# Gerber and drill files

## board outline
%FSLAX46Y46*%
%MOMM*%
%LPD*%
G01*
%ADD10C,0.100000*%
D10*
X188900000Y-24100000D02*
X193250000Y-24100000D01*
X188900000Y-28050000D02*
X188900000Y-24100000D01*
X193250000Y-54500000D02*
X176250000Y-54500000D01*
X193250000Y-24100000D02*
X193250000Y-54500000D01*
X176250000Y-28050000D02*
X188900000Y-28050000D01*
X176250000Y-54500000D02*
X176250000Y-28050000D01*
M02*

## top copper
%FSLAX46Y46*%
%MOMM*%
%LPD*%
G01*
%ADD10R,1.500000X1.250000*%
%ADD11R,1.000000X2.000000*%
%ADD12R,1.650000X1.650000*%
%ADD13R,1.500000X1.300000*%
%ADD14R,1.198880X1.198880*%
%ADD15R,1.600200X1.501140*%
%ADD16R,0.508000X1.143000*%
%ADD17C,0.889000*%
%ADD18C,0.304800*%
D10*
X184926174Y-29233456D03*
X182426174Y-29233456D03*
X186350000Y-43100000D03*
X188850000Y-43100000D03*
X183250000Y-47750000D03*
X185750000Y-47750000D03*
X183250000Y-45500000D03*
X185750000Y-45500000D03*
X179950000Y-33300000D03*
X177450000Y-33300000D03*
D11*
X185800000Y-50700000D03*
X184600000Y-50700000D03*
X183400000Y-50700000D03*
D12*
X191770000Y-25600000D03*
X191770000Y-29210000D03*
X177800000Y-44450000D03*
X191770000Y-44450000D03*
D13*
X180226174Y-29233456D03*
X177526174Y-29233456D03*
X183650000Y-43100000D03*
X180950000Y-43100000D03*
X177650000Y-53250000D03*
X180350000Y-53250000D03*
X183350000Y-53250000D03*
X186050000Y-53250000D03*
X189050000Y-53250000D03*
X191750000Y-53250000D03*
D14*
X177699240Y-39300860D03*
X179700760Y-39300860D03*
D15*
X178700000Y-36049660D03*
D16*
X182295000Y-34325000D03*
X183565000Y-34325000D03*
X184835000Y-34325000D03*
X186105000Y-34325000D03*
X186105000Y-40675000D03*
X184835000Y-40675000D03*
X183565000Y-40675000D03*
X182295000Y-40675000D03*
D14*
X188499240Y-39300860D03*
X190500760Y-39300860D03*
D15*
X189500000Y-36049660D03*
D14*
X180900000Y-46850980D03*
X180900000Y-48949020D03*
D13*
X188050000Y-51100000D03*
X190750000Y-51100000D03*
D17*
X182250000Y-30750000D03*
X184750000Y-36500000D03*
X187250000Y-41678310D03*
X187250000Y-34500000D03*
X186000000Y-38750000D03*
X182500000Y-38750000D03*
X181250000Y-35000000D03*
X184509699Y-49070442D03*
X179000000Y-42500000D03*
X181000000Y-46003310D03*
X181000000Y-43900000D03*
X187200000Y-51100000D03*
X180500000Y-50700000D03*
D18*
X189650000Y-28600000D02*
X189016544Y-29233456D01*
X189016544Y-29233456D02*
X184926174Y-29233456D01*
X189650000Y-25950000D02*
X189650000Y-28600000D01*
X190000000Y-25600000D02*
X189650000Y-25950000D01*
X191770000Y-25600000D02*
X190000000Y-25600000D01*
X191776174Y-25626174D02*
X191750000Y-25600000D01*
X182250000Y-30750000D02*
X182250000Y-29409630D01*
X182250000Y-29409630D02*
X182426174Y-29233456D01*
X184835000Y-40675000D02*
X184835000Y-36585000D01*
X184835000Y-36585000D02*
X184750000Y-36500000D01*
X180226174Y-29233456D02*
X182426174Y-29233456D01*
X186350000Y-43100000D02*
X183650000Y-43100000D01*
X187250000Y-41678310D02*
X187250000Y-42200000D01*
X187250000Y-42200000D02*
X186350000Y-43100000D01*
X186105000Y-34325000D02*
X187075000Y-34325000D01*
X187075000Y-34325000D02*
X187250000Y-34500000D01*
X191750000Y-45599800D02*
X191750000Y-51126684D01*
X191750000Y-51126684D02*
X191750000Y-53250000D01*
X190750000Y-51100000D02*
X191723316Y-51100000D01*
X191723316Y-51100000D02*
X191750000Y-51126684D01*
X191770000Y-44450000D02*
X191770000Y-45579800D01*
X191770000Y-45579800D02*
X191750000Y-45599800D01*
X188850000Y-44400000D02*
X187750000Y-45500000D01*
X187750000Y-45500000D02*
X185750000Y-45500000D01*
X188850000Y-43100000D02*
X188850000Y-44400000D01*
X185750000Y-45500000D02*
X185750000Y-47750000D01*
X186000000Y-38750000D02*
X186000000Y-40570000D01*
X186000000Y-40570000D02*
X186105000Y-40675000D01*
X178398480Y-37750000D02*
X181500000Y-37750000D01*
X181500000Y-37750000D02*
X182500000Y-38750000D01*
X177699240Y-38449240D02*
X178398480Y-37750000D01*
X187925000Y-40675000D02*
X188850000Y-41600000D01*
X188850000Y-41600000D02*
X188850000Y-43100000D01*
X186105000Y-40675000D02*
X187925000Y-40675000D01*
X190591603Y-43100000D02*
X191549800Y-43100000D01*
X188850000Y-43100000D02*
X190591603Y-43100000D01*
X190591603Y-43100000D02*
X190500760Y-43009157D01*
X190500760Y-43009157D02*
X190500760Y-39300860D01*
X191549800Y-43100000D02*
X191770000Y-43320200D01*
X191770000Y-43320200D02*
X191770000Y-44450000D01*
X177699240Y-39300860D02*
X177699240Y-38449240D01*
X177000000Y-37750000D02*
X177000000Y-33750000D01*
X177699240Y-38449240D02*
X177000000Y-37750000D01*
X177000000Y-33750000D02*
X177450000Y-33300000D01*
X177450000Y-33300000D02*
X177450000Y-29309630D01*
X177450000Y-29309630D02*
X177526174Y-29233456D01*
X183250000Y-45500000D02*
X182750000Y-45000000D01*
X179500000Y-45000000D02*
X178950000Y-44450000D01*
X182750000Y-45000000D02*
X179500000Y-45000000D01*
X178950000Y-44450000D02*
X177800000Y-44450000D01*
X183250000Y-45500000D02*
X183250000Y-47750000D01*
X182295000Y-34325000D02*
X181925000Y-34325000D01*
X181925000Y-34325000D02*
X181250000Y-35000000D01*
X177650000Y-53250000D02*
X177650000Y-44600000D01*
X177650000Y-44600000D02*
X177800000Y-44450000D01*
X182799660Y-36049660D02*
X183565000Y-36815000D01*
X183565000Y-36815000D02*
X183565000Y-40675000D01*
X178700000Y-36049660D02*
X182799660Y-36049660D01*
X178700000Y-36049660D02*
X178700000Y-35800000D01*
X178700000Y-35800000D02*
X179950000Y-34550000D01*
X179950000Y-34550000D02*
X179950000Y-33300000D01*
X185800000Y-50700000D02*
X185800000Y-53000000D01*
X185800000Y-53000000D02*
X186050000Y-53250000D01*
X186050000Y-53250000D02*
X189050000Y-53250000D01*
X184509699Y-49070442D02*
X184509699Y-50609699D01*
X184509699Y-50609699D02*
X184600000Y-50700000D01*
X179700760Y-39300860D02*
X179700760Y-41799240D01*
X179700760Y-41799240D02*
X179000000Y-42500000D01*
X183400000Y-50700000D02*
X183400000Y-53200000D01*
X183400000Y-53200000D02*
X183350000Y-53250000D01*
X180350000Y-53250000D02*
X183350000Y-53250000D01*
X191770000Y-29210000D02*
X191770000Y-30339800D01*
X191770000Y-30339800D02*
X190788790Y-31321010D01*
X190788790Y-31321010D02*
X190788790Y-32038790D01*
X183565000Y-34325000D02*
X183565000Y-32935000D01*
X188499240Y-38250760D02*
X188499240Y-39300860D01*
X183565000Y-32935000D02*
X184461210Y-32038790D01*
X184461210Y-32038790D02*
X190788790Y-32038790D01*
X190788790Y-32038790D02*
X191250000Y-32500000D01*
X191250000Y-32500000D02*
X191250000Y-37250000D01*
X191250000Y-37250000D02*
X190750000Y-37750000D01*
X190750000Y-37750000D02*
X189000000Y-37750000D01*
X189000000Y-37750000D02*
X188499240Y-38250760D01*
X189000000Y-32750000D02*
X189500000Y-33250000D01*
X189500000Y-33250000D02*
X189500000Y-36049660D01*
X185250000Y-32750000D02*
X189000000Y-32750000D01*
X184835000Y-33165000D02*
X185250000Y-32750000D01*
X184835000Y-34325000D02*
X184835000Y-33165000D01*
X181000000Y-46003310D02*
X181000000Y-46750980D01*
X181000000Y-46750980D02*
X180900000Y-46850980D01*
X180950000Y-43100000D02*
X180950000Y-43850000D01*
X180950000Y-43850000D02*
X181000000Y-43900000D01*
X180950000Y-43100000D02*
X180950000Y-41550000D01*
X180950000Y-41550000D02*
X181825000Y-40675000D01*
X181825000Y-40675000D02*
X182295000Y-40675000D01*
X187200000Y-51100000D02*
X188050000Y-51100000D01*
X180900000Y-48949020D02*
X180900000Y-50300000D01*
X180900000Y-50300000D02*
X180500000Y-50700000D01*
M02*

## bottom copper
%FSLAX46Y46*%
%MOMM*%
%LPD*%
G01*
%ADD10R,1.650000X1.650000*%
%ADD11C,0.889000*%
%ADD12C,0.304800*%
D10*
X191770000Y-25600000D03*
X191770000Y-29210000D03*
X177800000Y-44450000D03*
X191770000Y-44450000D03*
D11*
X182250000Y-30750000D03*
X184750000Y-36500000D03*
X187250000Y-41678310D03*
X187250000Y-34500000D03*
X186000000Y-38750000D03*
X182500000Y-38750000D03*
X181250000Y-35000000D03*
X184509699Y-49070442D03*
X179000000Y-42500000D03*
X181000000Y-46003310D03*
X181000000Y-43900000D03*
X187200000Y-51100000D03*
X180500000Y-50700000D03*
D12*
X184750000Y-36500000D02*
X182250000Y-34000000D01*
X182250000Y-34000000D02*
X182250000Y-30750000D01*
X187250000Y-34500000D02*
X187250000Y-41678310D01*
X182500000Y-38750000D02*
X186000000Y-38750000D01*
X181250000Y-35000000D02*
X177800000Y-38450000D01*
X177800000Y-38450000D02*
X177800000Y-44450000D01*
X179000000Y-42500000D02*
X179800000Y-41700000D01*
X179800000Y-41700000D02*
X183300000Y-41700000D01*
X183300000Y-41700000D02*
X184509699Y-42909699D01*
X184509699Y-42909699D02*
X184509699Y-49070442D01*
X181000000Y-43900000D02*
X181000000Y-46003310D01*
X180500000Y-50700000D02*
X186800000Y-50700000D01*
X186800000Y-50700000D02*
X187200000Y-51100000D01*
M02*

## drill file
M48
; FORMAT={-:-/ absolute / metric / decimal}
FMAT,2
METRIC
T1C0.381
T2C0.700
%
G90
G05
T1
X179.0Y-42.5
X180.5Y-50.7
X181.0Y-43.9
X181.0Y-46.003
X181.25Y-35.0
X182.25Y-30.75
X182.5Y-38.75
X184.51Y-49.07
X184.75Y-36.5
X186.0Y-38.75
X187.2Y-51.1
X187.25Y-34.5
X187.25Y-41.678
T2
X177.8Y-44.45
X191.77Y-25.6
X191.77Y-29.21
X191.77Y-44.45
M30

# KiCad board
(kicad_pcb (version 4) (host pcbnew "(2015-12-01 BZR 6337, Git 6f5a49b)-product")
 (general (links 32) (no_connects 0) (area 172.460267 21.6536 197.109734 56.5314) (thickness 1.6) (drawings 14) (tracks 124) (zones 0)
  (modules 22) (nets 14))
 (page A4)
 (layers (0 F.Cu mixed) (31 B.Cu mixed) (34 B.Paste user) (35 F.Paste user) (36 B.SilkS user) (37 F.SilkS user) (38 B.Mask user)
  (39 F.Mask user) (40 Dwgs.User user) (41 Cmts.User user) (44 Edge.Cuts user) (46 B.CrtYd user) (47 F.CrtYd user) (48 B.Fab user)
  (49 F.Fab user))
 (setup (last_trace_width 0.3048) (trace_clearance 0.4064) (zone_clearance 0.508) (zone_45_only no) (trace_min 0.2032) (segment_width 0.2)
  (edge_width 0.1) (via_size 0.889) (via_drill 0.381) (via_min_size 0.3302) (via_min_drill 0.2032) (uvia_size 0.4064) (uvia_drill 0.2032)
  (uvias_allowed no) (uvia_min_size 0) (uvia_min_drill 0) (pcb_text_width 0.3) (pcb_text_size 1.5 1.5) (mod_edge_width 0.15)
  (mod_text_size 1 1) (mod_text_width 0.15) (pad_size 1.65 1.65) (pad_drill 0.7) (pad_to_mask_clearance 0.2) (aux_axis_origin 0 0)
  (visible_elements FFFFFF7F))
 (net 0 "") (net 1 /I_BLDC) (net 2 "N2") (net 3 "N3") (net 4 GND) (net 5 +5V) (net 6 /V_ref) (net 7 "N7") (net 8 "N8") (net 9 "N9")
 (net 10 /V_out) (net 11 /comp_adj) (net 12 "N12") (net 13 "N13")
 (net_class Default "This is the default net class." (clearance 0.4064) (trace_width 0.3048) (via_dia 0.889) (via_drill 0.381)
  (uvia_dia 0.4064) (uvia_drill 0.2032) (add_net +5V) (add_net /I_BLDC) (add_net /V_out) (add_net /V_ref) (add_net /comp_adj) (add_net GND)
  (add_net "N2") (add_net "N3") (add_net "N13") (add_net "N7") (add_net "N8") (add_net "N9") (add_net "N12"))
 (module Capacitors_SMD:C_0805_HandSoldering (layer F.Cu) (at 183.676174 29.233456 180)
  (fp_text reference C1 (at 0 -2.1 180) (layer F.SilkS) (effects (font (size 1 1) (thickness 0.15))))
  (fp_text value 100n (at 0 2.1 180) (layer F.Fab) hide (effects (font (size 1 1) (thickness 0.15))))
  (pad 1 smd rect (at -1.25 0 180) (size 1.5 1.25) (layers F.Cu F.Paste F.Mask) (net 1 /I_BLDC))
  (pad 2 smd rect (at 1.25 0 180) (size 1.5 1.25) (layers F.Cu F.Paste F.Mask) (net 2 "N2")))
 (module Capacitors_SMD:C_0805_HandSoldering (layer F.Cu) (at 187.6 43.1)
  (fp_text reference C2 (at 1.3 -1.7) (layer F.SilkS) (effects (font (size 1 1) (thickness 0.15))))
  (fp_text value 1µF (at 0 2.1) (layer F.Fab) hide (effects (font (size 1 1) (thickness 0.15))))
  (pad 1 smd rect (at -1.25 0) (size 1.5 1.25) (layers F.Cu F.Paste F.Mask) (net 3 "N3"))
  (pad 2 smd rect (at 1.25 0) (size 1.5 1.25) (layers F.Cu F.Paste F.Mask) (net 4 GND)))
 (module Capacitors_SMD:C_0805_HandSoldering (layer F.Cu) (at 184.5 47.75)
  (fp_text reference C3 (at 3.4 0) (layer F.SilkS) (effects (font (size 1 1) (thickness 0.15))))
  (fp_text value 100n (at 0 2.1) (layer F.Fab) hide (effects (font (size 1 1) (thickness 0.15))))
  (pad 1 smd rect (at -1.25 0) (size 1.5 1.25) (layers F.Cu F.Paste F.Mask) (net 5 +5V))
  (pad 2 smd rect (at 1.25 0) (size 1.5 1.25) (layers F.Cu F.Paste F.Mask) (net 4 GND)))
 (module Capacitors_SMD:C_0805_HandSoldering (layer F.Cu) (at 184.5 45.5)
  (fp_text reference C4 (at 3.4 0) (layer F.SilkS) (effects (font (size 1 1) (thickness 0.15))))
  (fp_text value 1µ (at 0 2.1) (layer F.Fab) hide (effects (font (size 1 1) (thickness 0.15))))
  (pad 1 smd rect (at -1.25 0) (size 1.5 1.25) (layers F.Cu F.Paste F.Mask) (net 5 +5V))
  (pad 2 smd rect (at 1.25 0) (size 1.5 1.25) (layers F.Cu F.Paste F.Mask) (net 4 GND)))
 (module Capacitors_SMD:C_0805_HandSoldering (layer F.Cu) (at 178.7 33.3 180)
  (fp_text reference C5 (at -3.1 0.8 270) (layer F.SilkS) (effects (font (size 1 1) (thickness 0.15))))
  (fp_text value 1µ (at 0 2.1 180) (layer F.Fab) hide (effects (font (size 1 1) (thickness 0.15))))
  (pad 1 smd rect (at -1.25 0 180) (size 1.5 1.25) (layers F.Cu F.Paste F.Mask) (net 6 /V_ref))
  (pad 2 smd rect (at 1.25 0 180) (size 1.5 1.25) (layers F.Cu F.Paste F.Mask) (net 4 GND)))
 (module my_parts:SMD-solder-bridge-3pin (layer F.Cu) (at 184.6 50.7 180) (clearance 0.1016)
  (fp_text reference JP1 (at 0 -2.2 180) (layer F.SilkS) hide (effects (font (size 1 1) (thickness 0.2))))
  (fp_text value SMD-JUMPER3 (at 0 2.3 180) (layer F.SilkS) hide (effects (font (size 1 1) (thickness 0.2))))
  (pad 1 smd rect (at -1.2 0 180) (size 1 2) (layers F.Cu F.Mask) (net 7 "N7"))
  (pad 2 smd rect (at 0 0 180) (size 1 2) (layers F.Cu F.Mask) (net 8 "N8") (solder_mask_margin 0.3))
  (pad 3 smd rect (at 1.2 0 180) (size 1 2) (layers F.Cu F.Mask) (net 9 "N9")))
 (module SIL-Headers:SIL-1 (layer F.Cu) (at 191.77 25.6)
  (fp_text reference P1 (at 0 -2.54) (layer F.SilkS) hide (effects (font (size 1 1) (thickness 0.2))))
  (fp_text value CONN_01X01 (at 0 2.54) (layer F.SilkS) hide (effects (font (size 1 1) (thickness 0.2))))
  (pad 1 thru_hole rect (at 0 0) (size 1.65 1.65) (drill 0.7) (layers *.Cu *.Mask) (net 1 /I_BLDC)))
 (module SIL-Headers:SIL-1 (layer F.Cu) (at 191.77 29.21)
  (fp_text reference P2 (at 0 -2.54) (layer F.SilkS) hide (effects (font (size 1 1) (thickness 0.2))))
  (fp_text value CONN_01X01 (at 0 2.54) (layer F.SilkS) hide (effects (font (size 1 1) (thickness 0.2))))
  (pad 1 thru_hole rect (at 0 0) (size 1.65 1.65) (drill 0.7) (layers *.Cu *.Mask) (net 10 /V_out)))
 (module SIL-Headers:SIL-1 (layer F.Cu) (at 177.8 44.45)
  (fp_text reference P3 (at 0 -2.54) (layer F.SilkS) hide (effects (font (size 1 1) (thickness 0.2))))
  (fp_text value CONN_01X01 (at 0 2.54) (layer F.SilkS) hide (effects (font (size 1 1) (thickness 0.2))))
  (pad 1 thru_hole rect (at 0 0) (size 1.65 1.65) (drill 0.7) (layers *.Cu *.Mask) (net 5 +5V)))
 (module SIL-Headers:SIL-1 (layer F.Cu) (at 191.77 44.45)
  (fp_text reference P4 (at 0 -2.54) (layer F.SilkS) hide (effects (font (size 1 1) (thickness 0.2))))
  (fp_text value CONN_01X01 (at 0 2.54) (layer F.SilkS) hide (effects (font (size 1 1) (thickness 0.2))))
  (pad 1 thru_hole rect (at 0 0) (size 1.65 1.65) (drill 0.7) (layers *.Cu *.Mask) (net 4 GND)))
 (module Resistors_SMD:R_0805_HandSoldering (layer F.Cu) (at 178.876174 29.233456 180)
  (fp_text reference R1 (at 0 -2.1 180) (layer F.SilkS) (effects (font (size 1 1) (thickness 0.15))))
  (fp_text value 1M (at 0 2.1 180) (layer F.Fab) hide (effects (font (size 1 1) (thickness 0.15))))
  (pad 1 smd rect (at -1.35 0 180) (size 1.5 1.3) (layers F.Cu F.Paste F.Mask) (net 2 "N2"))
  (pad 2 smd rect (at 1.35 0 180) (size 1.5 1.3) (layers F.Cu F.Paste F.Mask) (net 4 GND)))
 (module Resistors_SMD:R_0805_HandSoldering (layer F.Cu) (at 182.3 43.1 180)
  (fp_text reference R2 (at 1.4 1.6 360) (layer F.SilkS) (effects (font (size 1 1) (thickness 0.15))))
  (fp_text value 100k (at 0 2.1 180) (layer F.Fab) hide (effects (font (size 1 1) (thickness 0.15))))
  (pad 1 smd rect (at -1.35 0 180) (size 1.5 1.3) (layers F.Cu F.Paste F.Mask) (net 3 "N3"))
  (pad 2 smd rect (at 1.35 0 180) (size 1.5 1.3) (layers F.Cu F.Paste F.Mask) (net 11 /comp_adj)))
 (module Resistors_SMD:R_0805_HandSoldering (layer F.Cu) (at 179 53.25)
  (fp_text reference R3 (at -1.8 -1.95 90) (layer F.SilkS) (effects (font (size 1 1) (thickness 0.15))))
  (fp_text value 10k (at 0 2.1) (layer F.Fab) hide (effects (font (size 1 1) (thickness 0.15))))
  (pad 1 smd rect (at -1.35 0) (size 1.5 1.3) (layers F.Cu F.Paste F.Mask) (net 5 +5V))
  (pad 2 smd rect (at 1.35 0) (size 1.5 1.3) (layers F.Cu F.Paste F.Mask) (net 9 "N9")))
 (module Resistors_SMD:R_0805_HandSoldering (layer F.Cu) (at 184.7 53.25)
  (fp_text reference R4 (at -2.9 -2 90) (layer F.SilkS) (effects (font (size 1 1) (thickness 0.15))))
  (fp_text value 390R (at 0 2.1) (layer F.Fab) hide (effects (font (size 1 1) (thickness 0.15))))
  (pad 1 smd rect (at -1.35 0) (size 1.5 1.3) (layers F.Cu F.Paste F.Mask) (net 9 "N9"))
  (pad 2 smd rect (at 1.35 0) (size 1.5 1.3) (layers F.Cu F.Paste F.Mask) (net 7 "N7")))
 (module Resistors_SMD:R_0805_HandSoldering (layer F.Cu) (at 190.4 53.25)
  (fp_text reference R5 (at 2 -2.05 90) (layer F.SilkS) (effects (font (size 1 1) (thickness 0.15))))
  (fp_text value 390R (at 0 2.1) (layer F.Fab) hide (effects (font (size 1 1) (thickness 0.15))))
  (pad 1 smd rect (at -1.35 0) (size 1.5 1.3) (layers F.Cu F.Paste F.Mask) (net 7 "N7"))
  (pad 2 smd rect (at 1.35 0) (size 1.5 1.3) (layers F.Cu F.Paste F.Mask) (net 4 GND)))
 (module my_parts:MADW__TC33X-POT (layer F.Cu) (at 178.7 37.5)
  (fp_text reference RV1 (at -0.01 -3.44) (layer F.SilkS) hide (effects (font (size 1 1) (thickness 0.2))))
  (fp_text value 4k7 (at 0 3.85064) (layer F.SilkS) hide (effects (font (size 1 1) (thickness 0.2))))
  (pad 1 smd rect (at -1.00076 1.80086) (size 1.19888 1.19888) (layers F.Cu F.Paste F.Mask) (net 4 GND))
  (pad 3 smd rect (at 1.00076 1.80086) (size 1.19888 1.19888) (layers F.Cu F.Paste F.Mask) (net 8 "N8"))
  (pad 2 smd rect (at 0 -1.45034) (size 1.6002 1.50114) (layers F.Cu F.Paste F.Mask) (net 6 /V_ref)))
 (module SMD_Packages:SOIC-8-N (layer F.Cu) (at 184.2 37.5)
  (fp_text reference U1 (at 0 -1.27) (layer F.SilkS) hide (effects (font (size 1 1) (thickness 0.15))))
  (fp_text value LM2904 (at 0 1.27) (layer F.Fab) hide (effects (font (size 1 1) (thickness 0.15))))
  (pad 8 smd rect (at -1.905 -3.175) (size 0.508 1.143) (layers F.Cu F.Paste F.Mask) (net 5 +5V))
  (pad 7 smd rect (at -0.635 -3.175) (size 0.508 1.143) (layers F.Cu F.Paste F.Mask) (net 10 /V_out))
  (pad 6 smd rect (at 0.635 -3.175) (size 0.508 1.143) (layers F.Cu F.Paste F.Mask) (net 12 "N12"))
  (pad 5 smd rect (at 1.905 -3.175) (size 0.508 1.143) (layers F.Cu F.Paste F.Mask) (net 3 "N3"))
  (pad 4 smd rect (at 1.905 3.175) (size 0.508 1.143) (layers F.Cu F.Paste F.Mask) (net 4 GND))
  (pad 3 smd rect (at 0.635 3.175) (size 0.508 1.143) (layers F.Cu F.Paste F.Mask) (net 2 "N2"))
  (pad 2 smd rect (at -0.635 3.175) (size 0.508 1.143) (layers F.Cu F.Paste F.Mask) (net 6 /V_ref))
  (pad 1 smd rect (at -1.905 3.175) (size 0.508 1.143) (layers F.Cu F.Paste F.Mask) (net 11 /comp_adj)))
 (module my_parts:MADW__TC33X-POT (layer F.Cu) (at 189.5 37.5)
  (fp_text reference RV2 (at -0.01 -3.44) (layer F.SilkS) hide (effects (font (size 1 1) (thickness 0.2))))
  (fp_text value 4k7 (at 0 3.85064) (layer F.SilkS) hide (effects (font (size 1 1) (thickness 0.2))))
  (pad 1 smd rect (at -1.00076 1.80086) (size 1.19888 1.19888) (layers F.Cu F.Paste F.Mask) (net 10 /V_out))
  (pad 3 smd rect (at 1.00076 1.80086) (size 1.19888 1.19888) (layers F.Cu F.Paste F.Mask) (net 4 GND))
  (pad 2 smd rect (at 0 -1.45034) (size 1.6002 1.50114) (layers F.Cu F.Paste F.Mask) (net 12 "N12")))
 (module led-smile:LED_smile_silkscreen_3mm (layer F.Cu) (at 186.85 31.85)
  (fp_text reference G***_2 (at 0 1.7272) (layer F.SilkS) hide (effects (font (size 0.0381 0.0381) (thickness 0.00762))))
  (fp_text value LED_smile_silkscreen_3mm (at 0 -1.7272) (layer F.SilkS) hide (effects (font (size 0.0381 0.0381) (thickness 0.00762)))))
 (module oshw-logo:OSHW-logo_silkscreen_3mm (layer F.Cu) (at 191.7 41.45)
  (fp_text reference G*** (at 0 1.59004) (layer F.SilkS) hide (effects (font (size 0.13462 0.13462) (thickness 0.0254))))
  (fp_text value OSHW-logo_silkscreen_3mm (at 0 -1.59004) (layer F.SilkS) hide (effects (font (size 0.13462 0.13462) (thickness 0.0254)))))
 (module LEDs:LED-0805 (layer F.Cu) (at 180.9 47.9 90)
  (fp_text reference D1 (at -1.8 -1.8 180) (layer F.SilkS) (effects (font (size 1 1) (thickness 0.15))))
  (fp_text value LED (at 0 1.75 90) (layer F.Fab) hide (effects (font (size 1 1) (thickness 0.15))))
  (pad 2 smd rect (at 1.04902 0 270) (size 1.19888 1.19888) (layers F.Cu F.Paste F.Mask) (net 11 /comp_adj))
  (pad 1 smd rect (at -1.04902 0 270) (size 1.19888 1.19888) (layers F.Cu F.Paste F.Mask) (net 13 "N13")))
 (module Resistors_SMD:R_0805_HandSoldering (layer F.Cu) (at 189.4 51.1)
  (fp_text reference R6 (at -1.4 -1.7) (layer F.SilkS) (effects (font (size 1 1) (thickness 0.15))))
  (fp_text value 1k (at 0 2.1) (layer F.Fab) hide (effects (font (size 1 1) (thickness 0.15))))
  (pad 1 smd rect (at -1.35 0) (size 1.5 1.3) (layers F.Cu F.Paste F.Mask) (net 13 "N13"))
  (pad 2 smd rect (at 1.35 0) (size 1.5 1.3) (layers F.Cu F.Paste F.Mask) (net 4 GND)))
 (gr_line (start 188.9 24.1) (end 193.25 24.1) (layer Edge.Cuts) (width 0.1))
 (gr_line (start 188.9 28.05) (end 188.9 24.1) (layer Edge.Cuts) (width 0.1))
 (gr_line (start 193.25 54.5) (end 176.25 54.5) (layer Edge.Cuts) (width 0.1))
 (gr_line (start 193.25 24.1) (end 193.25 54.5) (layer Edge.Cuts) (width 0.1))
 (gr_line (start 176.25 28.05) (end 188.9 28.05) (layer Edge.Cuts) (width 0.1))
 (gr_line (start 176.25 54.5) (end 176.25 28.05) (layer Edge.Cuts) (width 0.1))
 (segment (start 189.65 28.6) (end 189.016544 29.233456) (width 0.3048) (layer F.Cu) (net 1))
 (segment (start 189.016544 29.233456) (end 184.926174 29.233456) (width 0.3048) (layer F.Cu) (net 1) (status 20))
 (segment (start 189.65 25.95) (end 189.65 28.6) (width 0.3048) (layer F.Cu) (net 1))
 (segment (start 190 25.6) (end 189.65 25.95) (width 0.3048) (layer F.Cu) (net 1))
 (segment (start 191.77 25.6) (end 190 25.6) (width 0.3048) (layer F.Cu) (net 1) (status 10))
 (segment (start 191.776174 25.626174) (end 191.75 25.6) (width 0.3048) (layer F.Cu) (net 1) (status 30))
 (segment (start 182.25 30.75) (end 182.25 29.40963) (width 0.3048) (layer F.Cu) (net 2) (status 20))
 (segment (start 182.25 29.40963) (end 182.426174 29.233456) (width 0.3048) (layer F.Cu) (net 2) (status 30))
 (segment (start 184.75 36.5) (end 182.25 34) (width 0.3048) (layer B.Cu) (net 2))
 (segment (start 182.25 34) (end 182.25 30.75) (width 0.3048) (layer B.Cu) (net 2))
 (segment (start 184.835 40.675) (end 184.835 36.585) (width 0.3048) (layer F.Cu) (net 2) (status 10))
 (segment (start 184.835 36.585) (end 184.75 36.5) (width 0.3048) (layer F.Cu) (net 2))
 (segment (start 180.226174 29.233456) (end 182.426174 29.233456) (width 0.3048) (layer F.Cu) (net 2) (status 30))
 (segment (start 186.35 43.1) (end 183.65 43.1) (width 0.3048) (layer F.Cu) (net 3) (status 30))
 (segment (start 187.25 41.67831) (end 187.25 42.2) (width 0.3048) (layer F.Cu) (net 3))
 (segment (start 187.25 42.2) (end 186.35 43.1) (width 0.3048) (layer F.Cu) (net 3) (status 20))
 (segment (start 187.25 34.5) (end 187.25 41.67831) (width 0.3048) (layer B.Cu) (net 3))
 (segment (start 186.105 34.325) (end 187.075 34.325) (width 0.3048) (layer F.Cu) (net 3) (status 10))
 (segment (start 187.075 34.325) (end 187.25 34.5) (width 0.3048) (layer F.Cu) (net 3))
 (segment (start 191.75 45.5998) (end 191.75 51.126684) (width 0.3048) (layer F.Cu) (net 4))
 (segment (start 191.75 51.126684) (end 191.75 53.25) (width 0.3048) (layer F.Cu) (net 4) (status 20))
 (segment (start 190.75 51.1) (end 191.723316 51.1) (width 0.3048) (layer F.Cu) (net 4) (status 10))
 (segment (start 191.723316 51.1) (end 191.75 51.126684) (width 0.3048) (layer F.Cu) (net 4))
 (segment (start 191.77 44.45) (end 191.77 45.5798) (width 0.3048) (layer F.Cu) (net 4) (status 10))
 (segment (start 191.77 45.5798) (end 191.75 45.5998) (width 0.3048) (layer F.Cu) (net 4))
 (segment (start 188.85 44.4) (end 187.75 45.5) (width 0.3048) (layer F.Cu) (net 4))
 (segment (start 187.75 45.5) (end 185.75 45.5) (width 0.3048) (layer F.Cu) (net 4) (status 20))
 (segment (start 188.85 43.1) (end 188.85 44.4) (width 0.3048) (layer F.Cu) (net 4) (status 10))
 (segment (start 185.75 45.5) (end 185.75 47.75) (width 0.3048) (layer F.Cu) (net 4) (status 30))
 (segment (start 186 38.75) (end 186 40.57) (width 0.3048) (layer F.Cu) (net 4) (status 20))
 (segment (start 186 40.57) (end 186.105 40.675) (width 0.3048) (layer F.Cu) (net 4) (status 30))
 (segment (start 182.5 38.75) (end 186 38.75) (width 0.3048) (layer B.Cu) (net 4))
 (segment (start 178.39848 37.75) (end 181.5 37.75) (width 0.3048) (layer F.Cu) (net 4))
 (segment (start 181.5 37.75) (end 182.5 38.75) (width 0.3048) (layer F.Cu) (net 4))
 (segment (start 177.69924 38.44924) (end 178.39848 37.75) (width 0.3048) (layer F.Cu) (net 4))
 (segment (start 187.925 40.675) (end 188.85 41.6) (width 0.3048) (layer F.Cu) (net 4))
 (segment (start 188.85 41.6) (end 188.85 43.1) (width 0.3048) (layer F.Cu) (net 4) (status 20))
 (segment (start 186.105 40.675) (end 187.925 40.675) (width 0.3048) (layer F.Cu) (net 4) (status 10))
 (segment (start 190.591603 43.1) (end 191.5498 43.1) (width 0.3048) (layer F.Cu) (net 4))
 (segment (start 188.85 43.1) (end 190.591603 43.1) (width 0.3048) (layer F.Cu) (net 4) (status 10))
 (segment (start 190.591603 43.1) (end 190.50076 43.009157) (width 0.3048) (layer F.Cu) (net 4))
 (segment (start 190.50076 43.009157) (end 190.50076 39.30086) (width 0.3048) (layer F.Cu) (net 4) (status 20))
 (segment (start 191.5498 43.1) (end 191.77 43.3202) (width 0.3048) (layer F.Cu) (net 4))
 (segment (start 191.77 43.3202) (end 191.77 44.45) (width 0.3048) (layer F.Cu) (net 4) (status 20))
 (segment (start 177.69924 39.30086) (end 177.69924 38.44924) (width 0.3048) (layer F.Cu) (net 4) (status 10))
 (segment (start 177 37.75) (end 177 33.75) (width 0.3048) (layer F.Cu) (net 4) (status 20))
 (segment (start 177.69924 38.44924) (end 177 37.75) (width 0.3048) (layer F.Cu) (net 4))
 (segment (start 177 33.75) (end 177.45 33.3) (width 0.3048) (layer F.Cu) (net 4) (status 30))
 (segment (start 177.45 33.3) (end 177.45 29.30963) (width 0.3048) (layer F.Cu) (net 4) (status 30))
 (segment (start 177.45 29.30963) (end 177.526174 29.233456) (width 0.3048) (layer F.Cu) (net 4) (status 30))
 (segment (start 183.25 45.5) (end 182.75 45) (width 0.3048) (layer F.Cu) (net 5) (status 30))
 (segment (start 179.5 45) (end 178.95 44.45) (width 0.3048) (layer F.Cu) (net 5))
 (segment (start 182.75 45) (end 179.5 45) (width 0.3048) (layer F.Cu) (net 5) (status 10))
 (segment (start 178.95 44.45) (end 177.8 44.45) (width 0.3048) (layer F.Cu) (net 5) (status 20))
 (segment (start 183.25 45.5) (end 183.25 47.75) (width 0.3048) (layer F.Cu) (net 5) (status 30))
 (segment (start 181.25 35) (end 177.8 38.45) (width 0.3048) (layer B.Cu) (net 5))
 (segment (start 177.8 38.45) (end 177.8 44.45) (width 0.3048) (layer B.Cu) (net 5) (status 20))
 (segment (start 182.295 34.325) (end 181.925 34.325) (width 0.3048) (layer F.Cu) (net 5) (status 10))
 (segment (start 181.925 34.325) (end 181.25 35) (width 0.3048) (layer F.Cu) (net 5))
 (segment (start 177.65 53.25) (end 177.65 44.6) (width 0.3048) (layer F.Cu) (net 5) (status 30))
 (segment (start 177.65 44.6) (end 177.8 44.45) (width 0.3048) (layer F.Cu) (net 5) (status 30))
 (segment (start 182.79966 36.04966) (end 183.565 36.815) (width 0.3048) (layer F.Cu) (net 6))
 (segment (start 183.565 36.815) (end 183.565 40.675) (width 0.3048) (layer F.Cu) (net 6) (status 20))
 (segment (start 178.7 36.04966) (end 182.79966 36.04966) (width 0.3048) (layer F.Cu) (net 6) (status 10))
 (segment (start 178.7 36.04966) (end 178.7 35.8) (width 0.3048) (layer F.Cu) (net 6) (status 30))
 (segment (start 178.7 35.8) (end 179.95 34.55) (width 0.3048) (layer F.Cu) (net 6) (status 10))
 (segment (start 179.95 34.55) (end 179.95 33.3) (width 0.3048) (layer F.Cu) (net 6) (status 20))
 (segment (start 185.8 50.7) (end 185.8 53) (width 0.3048) (layer F.Cu) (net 7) (status 30))
 (segment (start 185.8 53) (end 186.05 53.25) (width 0.3048) (layer F.Cu) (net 7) (status 30))
 (segment (start 186.05 53.25) (end 189.05 53.25) (width 0.3048) (layer F.Cu) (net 7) (status 30))
 (segment (start 179 42.5) (end 179.8 41.7) (width 0.3048) (layer B.Cu) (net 8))
 (segment (start 179.8 41.7) (end 183.3 41.7) (width 0.3048) (layer B.Cu) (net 8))
 (segment (start 183.3 41.7) (end 184.509699 42.909699) (width 0.3048) (layer B.Cu) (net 8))
 (segment (start 184.509699 42.909699) (end 184.509699 49.070442) (width 0.3048) (layer B.Cu) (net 8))
 (segment (start 184.509699 49.070442) (end 184.509699 50.609699) (width 0.3048) (layer F.Cu) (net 8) (status 20))
 (segment (start 184.509699 50.609699) (end 184.6 50.7) (width 0.3048) (layer F.Cu) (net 8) (status 30))
 (segment (start 179.70076 39.30086) (end 179.70076 41.79924) (width 0.3048) (layer F.Cu) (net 8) (status 10))
 (segment (start 179.70076 41.79924) (end 179 42.5) (width 0.3048) (layer F.Cu) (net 8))
 (segment (start 183.4 50.7) (end 183.4 53.2) (width 0.3048) (layer F.Cu) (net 9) (status 30))
 (segment (start 183.4 53.2) (end 183.35 53.25) (width 0.3048) (layer F.Cu) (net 9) (status 30))
 (segment (start 180.35 53.25) (end 183.35 53.25) (width 0.3048) (layer F.Cu) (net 9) (status 30))
 (segment (start 191.77 29.21) (end 191.77 30.3398) (width 0.3048) (layer F.Cu) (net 10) (status 10))
 (segment (start 191.77 30.3398) (end 190.78879 31.32101) (width 0.3048) (layer F.Cu) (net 10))
 (segment (start 190.78879 31.32101) (end 190.78879 32.03879) (width 0.3048) (layer F.Cu) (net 10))
 (segment (start 183.565 34.325) (end 183.565 32.935) (width 0.3048) (layer F.Cu) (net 10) (status 10))
 (segment (start 188.49924 38.25076) (end 188.49924 39.30086) (width 0.3048) (layer F.Cu) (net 10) (status 20))
 (segment (start 183.565 32.935) (end 184.46121 32.03879) (width 0.3048) (layer F.Cu) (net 10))
 (segment (start 184.46121 32.03879) (end 190.78879 32.03879) (width 0.3048) (layer F.Cu) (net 10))
 (segment (start 190.78879 32.03879) (end 191.25 32.5) (width 0.3048) (layer F.Cu) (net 10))
 (segment (start 191.25 32.5) (end 191.25 37.25) (width 0.3048) (layer F.Cu) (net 10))
 (segment (start 191.25 37.25) (end 190.75 37.75) (width 0.3048) (layer F.Cu) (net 10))
 (segment (start 190.75 37.75) (end 189 37.75) (width 0.3048) (layer F.Cu) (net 10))
 (segment (start 189 37.75) (end 188.49924 38.25076) (width 0.3048) (layer F.Cu) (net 10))
 (segment (start 189 32.75) (end 189.5 33.25) (width 0.3048) (layer F.Cu) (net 12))
 (segment (start 189.5 33.25) (end 189.5 36.04966) (width 0.3048) (layer F.Cu) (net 12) (status 20))
 (segment (start 185.25 32.75) (end 189 32.75) (width 0.3048) (layer F.Cu) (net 12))
 (segment (start 184.835 33.165) (end 185.25 32.75) (width 0.3048) (layer F.Cu) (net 12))
 (segment (start 184.835 34.325) (end 184.835 33.165) (width 0.3048) (layer F.Cu) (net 12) (status 10))
 (segment (start 181 46.00331) (end 181 46.75098) (width 0.3048) (layer F.Cu) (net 11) (status 20))
 (segment (start 181 46.75098) (end 180.9 46.85098) (width 0.3048) (layer F.Cu) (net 11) (status 30))
 (segment (start 181 43.9) (end 181 46.00331) (width 0.3048) (layer B.Cu) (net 11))
 (segment (start 180.95 43.1) (end 180.95 43.85) (width 0.3048) (layer F.Cu) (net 11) (status 10))
 (segment (start 180.95 43.85) (end 181 43.9) (width 0.3048) (layer F.Cu) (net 11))
 (segment (start 180.95 43.1) (end 180.95 41.55) (width 0.3048) (layer F.Cu) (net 11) (status 10))
 (segment (start 180.95 41.55) (end 181.825 40.675) (width 0.3048) (layer F.Cu) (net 11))
 (segment (start 181.825 40.675) (end 182.295 40.675) (width 0.3048) (layer F.Cu) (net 11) (status 20))
 (segment (start 187.2 51.1) (end 188.05 51.1) (width 0.3048) (layer F.Cu) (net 13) (status 20))
 (segment (start 180.5 50.7) (end 186.8 50.7) (width 0.3048) (layer B.Cu) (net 13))
 (segment (start 186.8 50.7) (end 187.2 51.1) (width 0.3048) (layer B.Cu) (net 13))
 (segment (start 180.9 48.94902) (end 180.9 50.3) (width 0.3048) (layer F.Cu) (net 13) (status 10))
 (segment (start 180.9 50.3) (end 180.5 50.7) (width 0.3048) (layer F.Cu) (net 13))
 (via (at 182.25 30.75) (size 0.889) (drill 0.381) (layers F.Cu B.Cu) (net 2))
 (via (at 184.75 36.5) (size 0.889) (drill 0.381) (layers F.Cu B.Cu) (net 2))
 (via (at 187.25 41.67831) (size 0.889) (drill 0.381) (layers F.Cu B.Cu) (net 3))
 (via (at 187.25 34.5) (size 0.889) (drill 0.381) (layers F.Cu B.Cu) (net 3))
 (via (at 186 38.75) (size 0.889) (drill 0.381) (layers F.Cu B.Cu) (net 4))
 (via (at 182.5 38.75) (size 0.889) (drill 0.381) (layers F.Cu B.Cu) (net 4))
 (via (at 181.25 35) (size 0.889) (drill 0.381) (layers F.Cu B.Cu) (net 5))
 (via (at 184.509699 49.070442) (size 0.889) (drill 0.381) (layers F.Cu B.Cu) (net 8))
 (via (at 179 42.5) (size 0.889) (drill 0.381) (layers F.Cu B.Cu) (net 8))
 (via (at 181 46.00331) (size 0.889) (drill 0.381) (layers F.Cu B.Cu) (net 11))
 (via (at 181 43.9) (size 0.889) (drill 0.381) (layers F.Cu B.Cu) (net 11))
 (via (at 187.2 51.1) (size 0.889) (drill 0.381) (layers F.Cu B.Cu) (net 13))
 (via (at 180.5 50.7) (size 0.889) (drill 0.381) (layers F.Cu B.Cu) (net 13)))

